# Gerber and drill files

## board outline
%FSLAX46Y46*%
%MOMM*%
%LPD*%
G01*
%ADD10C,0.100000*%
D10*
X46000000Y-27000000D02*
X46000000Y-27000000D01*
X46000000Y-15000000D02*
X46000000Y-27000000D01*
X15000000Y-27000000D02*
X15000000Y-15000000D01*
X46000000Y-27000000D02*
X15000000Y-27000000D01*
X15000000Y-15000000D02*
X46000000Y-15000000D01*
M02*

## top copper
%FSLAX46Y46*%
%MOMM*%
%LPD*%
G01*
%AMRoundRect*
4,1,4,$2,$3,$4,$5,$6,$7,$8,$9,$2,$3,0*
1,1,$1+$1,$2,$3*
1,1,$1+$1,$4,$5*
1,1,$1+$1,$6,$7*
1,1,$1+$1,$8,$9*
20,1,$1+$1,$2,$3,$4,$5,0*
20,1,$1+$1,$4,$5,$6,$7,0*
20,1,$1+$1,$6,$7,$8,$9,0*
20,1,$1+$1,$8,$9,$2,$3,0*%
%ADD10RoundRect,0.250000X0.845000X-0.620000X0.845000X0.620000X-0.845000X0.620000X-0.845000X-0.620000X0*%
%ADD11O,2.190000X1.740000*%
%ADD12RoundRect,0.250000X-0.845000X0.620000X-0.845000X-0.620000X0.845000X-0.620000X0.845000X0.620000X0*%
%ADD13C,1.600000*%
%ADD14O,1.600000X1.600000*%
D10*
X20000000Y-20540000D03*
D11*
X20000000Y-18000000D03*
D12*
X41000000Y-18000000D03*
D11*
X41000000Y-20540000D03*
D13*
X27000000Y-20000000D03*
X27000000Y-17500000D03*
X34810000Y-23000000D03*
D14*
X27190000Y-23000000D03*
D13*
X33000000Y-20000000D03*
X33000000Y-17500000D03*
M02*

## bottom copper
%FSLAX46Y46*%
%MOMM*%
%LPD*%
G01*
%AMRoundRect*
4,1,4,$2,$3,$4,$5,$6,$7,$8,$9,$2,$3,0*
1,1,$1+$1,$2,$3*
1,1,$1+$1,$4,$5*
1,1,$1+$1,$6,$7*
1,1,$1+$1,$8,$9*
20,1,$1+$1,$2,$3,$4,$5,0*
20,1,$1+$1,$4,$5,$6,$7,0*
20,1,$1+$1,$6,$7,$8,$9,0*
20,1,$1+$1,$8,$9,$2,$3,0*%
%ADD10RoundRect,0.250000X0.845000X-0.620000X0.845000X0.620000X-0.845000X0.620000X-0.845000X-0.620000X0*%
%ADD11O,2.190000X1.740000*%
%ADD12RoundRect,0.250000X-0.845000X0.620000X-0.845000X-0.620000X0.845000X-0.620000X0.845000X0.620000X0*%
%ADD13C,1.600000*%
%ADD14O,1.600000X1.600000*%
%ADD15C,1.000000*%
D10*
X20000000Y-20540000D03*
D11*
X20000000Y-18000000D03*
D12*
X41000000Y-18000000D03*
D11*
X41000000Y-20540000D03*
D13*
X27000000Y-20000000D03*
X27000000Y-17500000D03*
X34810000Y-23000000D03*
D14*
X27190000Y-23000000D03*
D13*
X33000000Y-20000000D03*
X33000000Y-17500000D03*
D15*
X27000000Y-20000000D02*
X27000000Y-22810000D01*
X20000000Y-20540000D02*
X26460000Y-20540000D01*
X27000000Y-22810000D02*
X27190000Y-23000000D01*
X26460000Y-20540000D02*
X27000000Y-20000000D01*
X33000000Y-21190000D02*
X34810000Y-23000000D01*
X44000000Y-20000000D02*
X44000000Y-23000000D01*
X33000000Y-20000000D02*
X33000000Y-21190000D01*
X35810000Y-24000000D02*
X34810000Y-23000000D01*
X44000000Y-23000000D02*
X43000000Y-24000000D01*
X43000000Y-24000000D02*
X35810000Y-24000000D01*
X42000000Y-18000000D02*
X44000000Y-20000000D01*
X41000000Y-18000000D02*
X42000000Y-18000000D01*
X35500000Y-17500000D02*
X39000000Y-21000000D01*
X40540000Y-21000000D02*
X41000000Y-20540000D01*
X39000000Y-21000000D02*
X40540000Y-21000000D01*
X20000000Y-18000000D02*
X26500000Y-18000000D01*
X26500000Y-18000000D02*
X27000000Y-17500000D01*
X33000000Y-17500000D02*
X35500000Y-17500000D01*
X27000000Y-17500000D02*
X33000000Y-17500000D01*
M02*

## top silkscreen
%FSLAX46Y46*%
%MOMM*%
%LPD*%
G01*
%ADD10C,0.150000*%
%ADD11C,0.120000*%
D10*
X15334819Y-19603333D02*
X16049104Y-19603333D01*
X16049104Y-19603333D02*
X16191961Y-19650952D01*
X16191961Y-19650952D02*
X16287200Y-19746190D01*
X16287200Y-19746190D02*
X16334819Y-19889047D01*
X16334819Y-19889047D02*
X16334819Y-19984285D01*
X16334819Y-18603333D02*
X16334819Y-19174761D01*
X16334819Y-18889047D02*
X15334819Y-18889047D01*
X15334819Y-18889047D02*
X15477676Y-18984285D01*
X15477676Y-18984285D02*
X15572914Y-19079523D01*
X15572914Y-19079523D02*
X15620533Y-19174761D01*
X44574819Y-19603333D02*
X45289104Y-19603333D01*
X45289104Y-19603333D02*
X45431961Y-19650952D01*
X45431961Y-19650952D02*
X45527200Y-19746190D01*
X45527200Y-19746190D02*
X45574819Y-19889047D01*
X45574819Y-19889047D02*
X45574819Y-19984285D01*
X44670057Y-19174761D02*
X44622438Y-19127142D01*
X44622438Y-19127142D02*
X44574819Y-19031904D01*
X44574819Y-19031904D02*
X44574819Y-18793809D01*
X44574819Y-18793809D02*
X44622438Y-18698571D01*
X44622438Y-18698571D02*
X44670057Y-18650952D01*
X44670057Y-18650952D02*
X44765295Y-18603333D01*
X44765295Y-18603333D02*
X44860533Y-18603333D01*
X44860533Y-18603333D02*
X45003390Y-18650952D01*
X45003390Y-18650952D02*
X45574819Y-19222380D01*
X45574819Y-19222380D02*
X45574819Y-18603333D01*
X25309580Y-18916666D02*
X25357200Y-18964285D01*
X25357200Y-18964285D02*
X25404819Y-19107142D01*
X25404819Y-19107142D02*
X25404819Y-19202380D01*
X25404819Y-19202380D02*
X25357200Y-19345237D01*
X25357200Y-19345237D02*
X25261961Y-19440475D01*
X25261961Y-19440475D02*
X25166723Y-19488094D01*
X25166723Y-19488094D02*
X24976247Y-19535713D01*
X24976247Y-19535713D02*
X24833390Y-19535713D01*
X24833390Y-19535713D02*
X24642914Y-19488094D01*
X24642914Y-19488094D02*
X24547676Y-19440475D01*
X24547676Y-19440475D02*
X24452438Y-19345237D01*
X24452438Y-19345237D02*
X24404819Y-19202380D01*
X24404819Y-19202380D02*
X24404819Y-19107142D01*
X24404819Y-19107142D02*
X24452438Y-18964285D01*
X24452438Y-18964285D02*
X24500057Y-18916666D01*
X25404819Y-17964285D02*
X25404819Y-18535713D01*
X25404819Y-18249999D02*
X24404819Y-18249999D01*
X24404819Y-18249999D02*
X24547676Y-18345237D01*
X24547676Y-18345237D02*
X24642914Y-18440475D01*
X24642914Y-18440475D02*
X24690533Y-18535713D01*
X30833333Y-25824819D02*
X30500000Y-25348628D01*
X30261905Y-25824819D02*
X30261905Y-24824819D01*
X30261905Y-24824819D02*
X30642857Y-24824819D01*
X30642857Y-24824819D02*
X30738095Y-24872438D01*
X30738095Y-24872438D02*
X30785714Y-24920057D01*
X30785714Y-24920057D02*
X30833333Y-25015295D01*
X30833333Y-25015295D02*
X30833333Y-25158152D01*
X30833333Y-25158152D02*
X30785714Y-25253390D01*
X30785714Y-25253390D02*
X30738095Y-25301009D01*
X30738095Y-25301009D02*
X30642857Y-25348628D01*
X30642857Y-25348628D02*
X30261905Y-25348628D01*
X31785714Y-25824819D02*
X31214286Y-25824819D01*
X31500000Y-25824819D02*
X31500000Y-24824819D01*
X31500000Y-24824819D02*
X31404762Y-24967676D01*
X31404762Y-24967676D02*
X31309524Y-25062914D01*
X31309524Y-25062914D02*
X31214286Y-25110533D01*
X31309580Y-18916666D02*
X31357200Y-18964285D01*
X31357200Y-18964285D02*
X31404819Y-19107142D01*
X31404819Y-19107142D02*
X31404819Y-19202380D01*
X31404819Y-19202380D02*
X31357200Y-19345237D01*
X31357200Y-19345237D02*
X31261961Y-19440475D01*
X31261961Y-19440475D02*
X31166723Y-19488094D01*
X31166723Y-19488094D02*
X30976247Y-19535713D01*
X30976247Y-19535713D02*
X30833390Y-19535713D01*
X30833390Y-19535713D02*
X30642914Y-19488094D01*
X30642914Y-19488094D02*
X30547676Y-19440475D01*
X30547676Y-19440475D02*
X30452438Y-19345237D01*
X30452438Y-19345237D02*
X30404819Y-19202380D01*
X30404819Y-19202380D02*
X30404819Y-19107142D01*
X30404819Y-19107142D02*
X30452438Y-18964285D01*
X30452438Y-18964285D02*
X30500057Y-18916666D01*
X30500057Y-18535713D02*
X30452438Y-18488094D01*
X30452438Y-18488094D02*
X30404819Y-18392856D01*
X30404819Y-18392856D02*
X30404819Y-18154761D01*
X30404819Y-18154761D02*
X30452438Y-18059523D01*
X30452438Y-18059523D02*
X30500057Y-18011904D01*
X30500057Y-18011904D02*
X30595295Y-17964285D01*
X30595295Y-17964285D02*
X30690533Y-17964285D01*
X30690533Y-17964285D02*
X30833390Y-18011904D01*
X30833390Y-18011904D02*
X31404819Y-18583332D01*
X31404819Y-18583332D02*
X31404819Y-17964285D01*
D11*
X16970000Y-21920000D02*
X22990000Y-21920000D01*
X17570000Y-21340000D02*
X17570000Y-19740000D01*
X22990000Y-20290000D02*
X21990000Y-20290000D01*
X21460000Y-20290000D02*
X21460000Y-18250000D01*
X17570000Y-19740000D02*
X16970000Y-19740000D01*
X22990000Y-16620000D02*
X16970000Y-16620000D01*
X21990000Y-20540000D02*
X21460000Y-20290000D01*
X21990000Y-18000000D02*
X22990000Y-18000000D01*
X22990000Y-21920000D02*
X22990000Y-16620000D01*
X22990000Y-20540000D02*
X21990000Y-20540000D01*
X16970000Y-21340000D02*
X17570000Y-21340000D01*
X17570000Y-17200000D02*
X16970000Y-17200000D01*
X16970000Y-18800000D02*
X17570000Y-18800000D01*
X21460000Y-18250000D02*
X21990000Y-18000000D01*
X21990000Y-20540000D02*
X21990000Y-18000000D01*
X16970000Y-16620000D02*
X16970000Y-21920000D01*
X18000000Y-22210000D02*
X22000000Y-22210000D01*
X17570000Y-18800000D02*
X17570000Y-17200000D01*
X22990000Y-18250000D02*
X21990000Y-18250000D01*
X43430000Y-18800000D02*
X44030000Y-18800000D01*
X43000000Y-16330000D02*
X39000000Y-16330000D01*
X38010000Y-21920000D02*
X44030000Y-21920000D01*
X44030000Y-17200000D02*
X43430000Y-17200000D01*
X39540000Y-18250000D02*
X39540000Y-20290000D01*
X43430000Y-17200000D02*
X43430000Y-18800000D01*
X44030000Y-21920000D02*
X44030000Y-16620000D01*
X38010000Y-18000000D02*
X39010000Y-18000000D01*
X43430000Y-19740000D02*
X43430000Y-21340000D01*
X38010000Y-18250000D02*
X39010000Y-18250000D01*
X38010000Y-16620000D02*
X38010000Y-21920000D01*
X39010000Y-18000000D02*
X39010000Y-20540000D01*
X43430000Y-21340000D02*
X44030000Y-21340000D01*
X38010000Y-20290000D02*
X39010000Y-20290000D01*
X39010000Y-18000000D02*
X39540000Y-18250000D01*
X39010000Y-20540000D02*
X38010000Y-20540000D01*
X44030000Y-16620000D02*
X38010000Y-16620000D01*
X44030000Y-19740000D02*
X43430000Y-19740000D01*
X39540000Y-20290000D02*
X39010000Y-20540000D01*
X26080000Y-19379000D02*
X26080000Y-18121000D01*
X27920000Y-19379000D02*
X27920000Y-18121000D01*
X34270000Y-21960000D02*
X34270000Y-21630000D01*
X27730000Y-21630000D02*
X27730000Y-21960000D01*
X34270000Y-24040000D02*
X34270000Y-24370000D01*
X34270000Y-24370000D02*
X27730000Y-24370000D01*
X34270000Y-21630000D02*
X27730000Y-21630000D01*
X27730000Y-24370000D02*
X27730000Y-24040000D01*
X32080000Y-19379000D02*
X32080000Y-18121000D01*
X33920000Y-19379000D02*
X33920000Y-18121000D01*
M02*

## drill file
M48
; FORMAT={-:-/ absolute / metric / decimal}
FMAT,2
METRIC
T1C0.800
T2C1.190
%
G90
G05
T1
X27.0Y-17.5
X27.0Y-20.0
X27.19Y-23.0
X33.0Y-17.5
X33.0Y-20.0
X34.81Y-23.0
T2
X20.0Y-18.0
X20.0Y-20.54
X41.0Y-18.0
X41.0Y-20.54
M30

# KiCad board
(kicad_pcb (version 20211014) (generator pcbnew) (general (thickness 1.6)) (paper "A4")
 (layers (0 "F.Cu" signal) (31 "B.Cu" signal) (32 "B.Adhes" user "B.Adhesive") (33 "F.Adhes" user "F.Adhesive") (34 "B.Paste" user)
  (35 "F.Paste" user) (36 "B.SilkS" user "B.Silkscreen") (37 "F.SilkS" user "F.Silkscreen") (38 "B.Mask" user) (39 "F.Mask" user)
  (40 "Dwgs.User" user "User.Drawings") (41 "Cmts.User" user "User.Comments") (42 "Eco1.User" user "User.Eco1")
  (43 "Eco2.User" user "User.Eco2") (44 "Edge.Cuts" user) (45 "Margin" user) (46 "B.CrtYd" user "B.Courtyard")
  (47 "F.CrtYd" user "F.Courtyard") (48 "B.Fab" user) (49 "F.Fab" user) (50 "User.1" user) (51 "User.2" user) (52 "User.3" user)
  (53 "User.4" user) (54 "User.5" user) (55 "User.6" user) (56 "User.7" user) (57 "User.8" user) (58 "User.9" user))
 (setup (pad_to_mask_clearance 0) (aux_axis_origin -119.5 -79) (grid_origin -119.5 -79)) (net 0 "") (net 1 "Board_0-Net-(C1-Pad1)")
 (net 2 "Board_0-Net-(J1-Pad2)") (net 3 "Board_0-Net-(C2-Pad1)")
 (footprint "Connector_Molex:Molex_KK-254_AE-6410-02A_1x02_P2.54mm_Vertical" (layer "F.Cu") (at 20 20.54 90)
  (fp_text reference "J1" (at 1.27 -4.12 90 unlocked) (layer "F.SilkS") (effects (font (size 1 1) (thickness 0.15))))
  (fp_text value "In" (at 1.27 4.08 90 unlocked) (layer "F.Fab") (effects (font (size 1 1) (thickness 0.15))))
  (fp_line (start -1.38 -3.03) (end -1.38 2.99) (layer "F.SilkS") (width 0.12))
  (fp_line (start -0.8 -2.43) (end 0.8 -2.43) (layer "F.SilkS") (width 0.12))
  (fp_line (start 0.25 2.99) (end 0.25 1.99) (layer "F.SilkS") (width 0.12))
  (fp_line (start 0.25 1.46) (end 2.29 1.46) (layer "F.SilkS") (width 0.12))
  (fp_line (start 0.8 -2.43) (end 0.8 -3.03) (layer "F.SilkS") (width 0.12))
  (fp_line (start 3.92 2.99) (end 3.92 -3.03) (layer "F.SilkS") (width 0.12))
  (fp_line (start 0 1.99) (end 0.25 1.46) (layer "F.SilkS") (width 0.12))
  (fp_line (start 2.54 1.99) (end 2.54 2.99) (layer "F.SilkS") (width 0.12))
  (fp_line (start -1.38 2.99) (end 3.92 2.99) (layer "F.SilkS") (width 0.12))
  (fp_line (start 0 2.99) (end 0 1.99) (layer "F.SilkS") (width 0.12))
  (fp_line (start -0.8 -3.03) (end -0.8 -2.43) (layer "F.SilkS") (width 0.12))
  (fp_line (start 3.34 -2.43) (end 3.34 -3.03) (layer "F.SilkS") (width 0.12))
  (fp_line (start 1.74 -3.03) (end 1.74 -2.43) (layer "F.SilkS") (width 0.12))
  (fp_line (start 2.29 1.46) (end 2.54 1.99) (layer "F.SilkS") (width 0.12))
  (fp_line (start 0 1.99) (end 2.54 1.99) (layer "F.SilkS") (width 0.12))
  (fp_line (start 3.92 -3.03) (end -1.38 -3.03) (layer "F.SilkS") (width 0.12))
  (fp_line (start -1.67 -2) (end -1.67 2) (layer "F.SilkS") (width 0.12))
  (fp_line (start 1.74 -2.43) (end 3.34 -2.43) (layer "F.SilkS") (width 0.12))
  (fp_line (start 2.29 2.99) (end 2.29 1.99) (layer "F.SilkS") (width 0.12))
  (pad "1" thru_hole roundrect (at 0 0 90) (size 1.74 2.19) (drill 1.19) (layers *.Cu *.Mask) (roundrect_rratio 0.143678)
   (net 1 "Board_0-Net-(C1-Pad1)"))
  (pad "2" thru_hole oval (at 2.54 0 90) (size 1.74 2.19) (drill 1.19) (layers *.Cu *.Mask) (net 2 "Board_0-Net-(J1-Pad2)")))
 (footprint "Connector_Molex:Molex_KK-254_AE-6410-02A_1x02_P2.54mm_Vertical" (layer "F.Cu") (at 41 18 -90)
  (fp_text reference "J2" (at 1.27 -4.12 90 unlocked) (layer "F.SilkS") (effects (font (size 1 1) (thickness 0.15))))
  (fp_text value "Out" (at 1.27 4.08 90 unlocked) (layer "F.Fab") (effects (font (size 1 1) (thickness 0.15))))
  (fp_line (start 0.8 -2.43) (end 0.8 -3.03) (layer "F.SilkS") (width 0.12))
  (fp_line (start -1.67 -2) (end -1.67 2) (layer "F.SilkS") (width 0.12))
  (fp_line (start 3.92 2.99) (end 3.92 -3.03) (layer "F.SilkS") (width 0.12))
  (fp_line (start -0.8 -3.03) (end -0.8 -2.43) (layer "F.SilkS") (width 0.12))
  (fp_line (start 0.25 1.46) (end 2.29 1.46) (layer "F.SilkS") (width 0.12))
  (fp_line (start -0.8 -2.43) (end 0.8 -2.43) (layer "F.SilkS") (width 0.12))
  (fp_line (start 3.92 -3.03) (end -1.38 -3.03) (layer "F.SilkS") (width 0.12))
  (fp_line (start 0 2.99) (end 0 1.99) (layer "F.SilkS") (width 0.12))
  (fp_line (start 1.74 -2.43) (end 3.34 -2.43) (layer "F.SilkS") (width 0.12))
  (fp_line (start 0.25 2.99) (end 0.25 1.99) (layer "F.SilkS") (width 0.12))
  (fp_line (start -1.38 2.99) (end 3.92 2.99) (layer "F.SilkS") (width 0.12))
  (fp_line (start 0 1.99) (end 2.54 1.99) (layer "F.SilkS") (width 0.12))
  (fp_line (start 3.34 -2.43) (end 3.34 -3.03) (layer "F.SilkS") (width 0.12))
  (fp_line (start 2.29 2.99) (end 2.29 1.99) (layer "F.SilkS") (width 0.12))
  (fp_line (start 0 1.99) (end 0.25 1.46) (layer "F.SilkS") (width 0.12))
  (fp_line (start 2.54 1.99) (end 2.54 2.99) (layer "F.SilkS") (width 0.12))
  (fp_line (start -1.38 -3.03) (end -1.38 2.99) (layer "F.SilkS") (width 0.12))
  (fp_line (start 1.74 -3.03) (end 1.74 -2.43) (layer "F.SilkS") (width 0.12))
  (fp_line (start 2.29 1.46) (end 2.54 1.99) (layer "F.SilkS") (width 0.12))
  (pad "1" thru_hole roundrect (at 0 0 270) (size 1.74 2.19) (drill 1.19) (layers *.Cu *.Mask) (roundrect_rratio 0.143678)
   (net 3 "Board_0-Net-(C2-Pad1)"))
  (pad "2" thru_hole oval (at 2.54 0 270) (size 1.74 2.19) (drill 1.19) (layers *.Cu *.Mask) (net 2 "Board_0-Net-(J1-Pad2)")))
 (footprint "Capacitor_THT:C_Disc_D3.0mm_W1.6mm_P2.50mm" (layer "F.Cu") (at 27 20 90)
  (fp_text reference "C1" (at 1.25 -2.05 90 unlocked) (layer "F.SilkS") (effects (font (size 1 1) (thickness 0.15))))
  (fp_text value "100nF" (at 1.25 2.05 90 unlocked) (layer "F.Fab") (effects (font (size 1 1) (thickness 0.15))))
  (fp_line (start 0.621 -0.92) (end 1.879 -0.92) (layer "F.SilkS") (width 0.12))
  (fp_line (start 0.621 0.92) (end 1.879 0.92) (layer "F.SilkS") (width 0.12))
  (pad "1" thru_hole circle (at 0 0 90) (size 1.6 1.6) (drill 0.8) (layers *.Cu *.Mask) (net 1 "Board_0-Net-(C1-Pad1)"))
  (pad "2" thru_hole circle (at 2.5 0 90) (size 1.6 1.6) (drill 0.8) (layers *.Cu *.Mask) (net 2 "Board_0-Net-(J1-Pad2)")))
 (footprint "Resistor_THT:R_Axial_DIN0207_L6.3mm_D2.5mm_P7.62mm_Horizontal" (layer "F.Cu") (at 34.81 23 180)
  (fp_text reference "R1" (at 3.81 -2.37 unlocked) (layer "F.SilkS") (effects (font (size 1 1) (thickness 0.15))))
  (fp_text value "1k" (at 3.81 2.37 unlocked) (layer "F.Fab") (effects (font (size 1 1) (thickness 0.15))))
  (fp_line (start 0.54 1.04) (end 0.54 1.37) (layer "F.SilkS") (width 0.12))
  (fp_line (start 7.08 1.37) (end 7.08 1.04) (layer "F.SilkS") (width 0.12))
  (fp_line (start 0.54 -1.04) (end 0.54 -1.37) (layer "F.SilkS") (width 0.12))
  (fp_line (start 0.54 -1.37) (end 7.08 -1.37) (layer "F.SilkS") (width 0.12))
  (fp_line (start 0.54 1.37) (end 7.08 1.37) (layer "F.SilkS") (width 0.12))
  (fp_line (start 7.08 -1.37) (end 7.08 -1.04) (layer "F.SilkS") (width 0.12))
  (pad "1" thru_hole circle (at 0 0 180) (size 1.6 1.6) (drill 0.8) (layers *.Cu *.Mask) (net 3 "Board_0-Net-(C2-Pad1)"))
  (pad "2" thru_hole oval (at 7.62 0 180) (size 1.6 1.6) (drill 0.8) (layers *.Cu *.Mask) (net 1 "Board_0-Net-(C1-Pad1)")))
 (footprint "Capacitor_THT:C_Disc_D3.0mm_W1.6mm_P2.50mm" (layer "F.Cu") (at 33 20 90)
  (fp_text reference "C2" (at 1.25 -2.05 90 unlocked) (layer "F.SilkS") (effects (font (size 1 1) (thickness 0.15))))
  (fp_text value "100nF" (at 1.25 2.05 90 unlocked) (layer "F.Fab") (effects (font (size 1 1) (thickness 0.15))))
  (fp_line (start 0.621 -0.92) (end 1.879 -0.92) (layer "F.SilkS") (width 0.12))
  (fp_line (start 0.621 0.92) (end 1.879 0.92) (layer "F.SilkS") (width 0.12))
  (pad "1" thru_hole circle (at 0 0 90) (size 1.6 1.6) (drill 0.8) (layers *.Cu *.Mask) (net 3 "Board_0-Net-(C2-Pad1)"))
  (pad "2" thru_hole circle (at 2.5 0 90) (size 1.6 1.6) (drill 0.8) (layers *.Cu *.Mask) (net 2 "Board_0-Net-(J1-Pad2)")))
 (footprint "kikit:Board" (layer "F.Cu") (at 17 15)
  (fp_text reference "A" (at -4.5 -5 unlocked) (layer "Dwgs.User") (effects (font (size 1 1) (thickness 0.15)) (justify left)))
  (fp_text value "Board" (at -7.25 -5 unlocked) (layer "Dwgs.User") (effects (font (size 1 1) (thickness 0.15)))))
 (gr_line (start 46 27) (end 46 27) (layer "Edge.Cuts") (width 0.1))
 (gr_line (start 46 15) (end 46 27) (layer "Edge.Cuts") (width 0.1))
 (gr_line (start 15 27) (end 15 15) (layer "Edge.Cuts") (width 0.1))
 (gr_line (start 46 27) (end 15 27) (layer "Edge.Cuts") (width 0.1))
 (gr_line (start 15 15) (end 46 15) (layer "Edge.Cuts") (width 0.1))
 (segment (start 27 20) (end 27 22.81) (width 1) (layer "B.Cu") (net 1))
 (segment (start 20 20.54) (end 26.46 20.54) (width 1) (layer "B.Cu") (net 1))
 (segment (start 27 22.81) (end 27.19 23) (width 1) (layer "B.Cu") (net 1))
 (segment (start 26.46 20.54) (end 27 20) (width 1) (layer "B.Cu") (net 1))
 (segment (start 33 21.19) (end 34.81 23) (width 1) (layer "B.Cu") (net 3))
 (segment (start 44 20) (end 44 23) (width 1) (layer "B.Cu") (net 3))
 (segment (start 33 20) (end 33 21.19) (width 1) (layer "B.Cu") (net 3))
 (segment (start 35.81 24) (end 34.81 23) (width 1) (layer "B.Cu") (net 3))
 (segment (start 44 23) (end 43 24) (width 1) (layer "B.Cu") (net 3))
 (segment (start 43 24) (end 35.81 24) (width 1) (layer "B.Cu") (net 3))
 (segment (start 42 18) (end 44 20) (width 1) (layer "B.Cu") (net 3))
 (segment (start 41 18) (end 42 18) (width 1) (layer "B.Cu") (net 3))
 (segment (start 35.5 17.5) (end 39 21) (width 1) (layer "B.Cu") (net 2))
 (segment (start 40.54 21) (end 41 20.54) (width 1) (layer "B.Cu") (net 2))
 (segment (start 39 21) (end 40.54 21) (width 1) (layer "B.Cu") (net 2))
 (segment (start 20 18) (end 26.5 18) (width 1) (layer "B.Cu") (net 2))
 (segment (start 26.5 18) (end 27 17.5) (width 1) (layer "B.Cu") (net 2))
 (segment (start 33 17.5) (end 35.5 17.5) (width 1) (layer "B.Cu") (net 2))
 (segment (start 27 17.5) (end 33 17.5) (width 1) (layer "B.Cu") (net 2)))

